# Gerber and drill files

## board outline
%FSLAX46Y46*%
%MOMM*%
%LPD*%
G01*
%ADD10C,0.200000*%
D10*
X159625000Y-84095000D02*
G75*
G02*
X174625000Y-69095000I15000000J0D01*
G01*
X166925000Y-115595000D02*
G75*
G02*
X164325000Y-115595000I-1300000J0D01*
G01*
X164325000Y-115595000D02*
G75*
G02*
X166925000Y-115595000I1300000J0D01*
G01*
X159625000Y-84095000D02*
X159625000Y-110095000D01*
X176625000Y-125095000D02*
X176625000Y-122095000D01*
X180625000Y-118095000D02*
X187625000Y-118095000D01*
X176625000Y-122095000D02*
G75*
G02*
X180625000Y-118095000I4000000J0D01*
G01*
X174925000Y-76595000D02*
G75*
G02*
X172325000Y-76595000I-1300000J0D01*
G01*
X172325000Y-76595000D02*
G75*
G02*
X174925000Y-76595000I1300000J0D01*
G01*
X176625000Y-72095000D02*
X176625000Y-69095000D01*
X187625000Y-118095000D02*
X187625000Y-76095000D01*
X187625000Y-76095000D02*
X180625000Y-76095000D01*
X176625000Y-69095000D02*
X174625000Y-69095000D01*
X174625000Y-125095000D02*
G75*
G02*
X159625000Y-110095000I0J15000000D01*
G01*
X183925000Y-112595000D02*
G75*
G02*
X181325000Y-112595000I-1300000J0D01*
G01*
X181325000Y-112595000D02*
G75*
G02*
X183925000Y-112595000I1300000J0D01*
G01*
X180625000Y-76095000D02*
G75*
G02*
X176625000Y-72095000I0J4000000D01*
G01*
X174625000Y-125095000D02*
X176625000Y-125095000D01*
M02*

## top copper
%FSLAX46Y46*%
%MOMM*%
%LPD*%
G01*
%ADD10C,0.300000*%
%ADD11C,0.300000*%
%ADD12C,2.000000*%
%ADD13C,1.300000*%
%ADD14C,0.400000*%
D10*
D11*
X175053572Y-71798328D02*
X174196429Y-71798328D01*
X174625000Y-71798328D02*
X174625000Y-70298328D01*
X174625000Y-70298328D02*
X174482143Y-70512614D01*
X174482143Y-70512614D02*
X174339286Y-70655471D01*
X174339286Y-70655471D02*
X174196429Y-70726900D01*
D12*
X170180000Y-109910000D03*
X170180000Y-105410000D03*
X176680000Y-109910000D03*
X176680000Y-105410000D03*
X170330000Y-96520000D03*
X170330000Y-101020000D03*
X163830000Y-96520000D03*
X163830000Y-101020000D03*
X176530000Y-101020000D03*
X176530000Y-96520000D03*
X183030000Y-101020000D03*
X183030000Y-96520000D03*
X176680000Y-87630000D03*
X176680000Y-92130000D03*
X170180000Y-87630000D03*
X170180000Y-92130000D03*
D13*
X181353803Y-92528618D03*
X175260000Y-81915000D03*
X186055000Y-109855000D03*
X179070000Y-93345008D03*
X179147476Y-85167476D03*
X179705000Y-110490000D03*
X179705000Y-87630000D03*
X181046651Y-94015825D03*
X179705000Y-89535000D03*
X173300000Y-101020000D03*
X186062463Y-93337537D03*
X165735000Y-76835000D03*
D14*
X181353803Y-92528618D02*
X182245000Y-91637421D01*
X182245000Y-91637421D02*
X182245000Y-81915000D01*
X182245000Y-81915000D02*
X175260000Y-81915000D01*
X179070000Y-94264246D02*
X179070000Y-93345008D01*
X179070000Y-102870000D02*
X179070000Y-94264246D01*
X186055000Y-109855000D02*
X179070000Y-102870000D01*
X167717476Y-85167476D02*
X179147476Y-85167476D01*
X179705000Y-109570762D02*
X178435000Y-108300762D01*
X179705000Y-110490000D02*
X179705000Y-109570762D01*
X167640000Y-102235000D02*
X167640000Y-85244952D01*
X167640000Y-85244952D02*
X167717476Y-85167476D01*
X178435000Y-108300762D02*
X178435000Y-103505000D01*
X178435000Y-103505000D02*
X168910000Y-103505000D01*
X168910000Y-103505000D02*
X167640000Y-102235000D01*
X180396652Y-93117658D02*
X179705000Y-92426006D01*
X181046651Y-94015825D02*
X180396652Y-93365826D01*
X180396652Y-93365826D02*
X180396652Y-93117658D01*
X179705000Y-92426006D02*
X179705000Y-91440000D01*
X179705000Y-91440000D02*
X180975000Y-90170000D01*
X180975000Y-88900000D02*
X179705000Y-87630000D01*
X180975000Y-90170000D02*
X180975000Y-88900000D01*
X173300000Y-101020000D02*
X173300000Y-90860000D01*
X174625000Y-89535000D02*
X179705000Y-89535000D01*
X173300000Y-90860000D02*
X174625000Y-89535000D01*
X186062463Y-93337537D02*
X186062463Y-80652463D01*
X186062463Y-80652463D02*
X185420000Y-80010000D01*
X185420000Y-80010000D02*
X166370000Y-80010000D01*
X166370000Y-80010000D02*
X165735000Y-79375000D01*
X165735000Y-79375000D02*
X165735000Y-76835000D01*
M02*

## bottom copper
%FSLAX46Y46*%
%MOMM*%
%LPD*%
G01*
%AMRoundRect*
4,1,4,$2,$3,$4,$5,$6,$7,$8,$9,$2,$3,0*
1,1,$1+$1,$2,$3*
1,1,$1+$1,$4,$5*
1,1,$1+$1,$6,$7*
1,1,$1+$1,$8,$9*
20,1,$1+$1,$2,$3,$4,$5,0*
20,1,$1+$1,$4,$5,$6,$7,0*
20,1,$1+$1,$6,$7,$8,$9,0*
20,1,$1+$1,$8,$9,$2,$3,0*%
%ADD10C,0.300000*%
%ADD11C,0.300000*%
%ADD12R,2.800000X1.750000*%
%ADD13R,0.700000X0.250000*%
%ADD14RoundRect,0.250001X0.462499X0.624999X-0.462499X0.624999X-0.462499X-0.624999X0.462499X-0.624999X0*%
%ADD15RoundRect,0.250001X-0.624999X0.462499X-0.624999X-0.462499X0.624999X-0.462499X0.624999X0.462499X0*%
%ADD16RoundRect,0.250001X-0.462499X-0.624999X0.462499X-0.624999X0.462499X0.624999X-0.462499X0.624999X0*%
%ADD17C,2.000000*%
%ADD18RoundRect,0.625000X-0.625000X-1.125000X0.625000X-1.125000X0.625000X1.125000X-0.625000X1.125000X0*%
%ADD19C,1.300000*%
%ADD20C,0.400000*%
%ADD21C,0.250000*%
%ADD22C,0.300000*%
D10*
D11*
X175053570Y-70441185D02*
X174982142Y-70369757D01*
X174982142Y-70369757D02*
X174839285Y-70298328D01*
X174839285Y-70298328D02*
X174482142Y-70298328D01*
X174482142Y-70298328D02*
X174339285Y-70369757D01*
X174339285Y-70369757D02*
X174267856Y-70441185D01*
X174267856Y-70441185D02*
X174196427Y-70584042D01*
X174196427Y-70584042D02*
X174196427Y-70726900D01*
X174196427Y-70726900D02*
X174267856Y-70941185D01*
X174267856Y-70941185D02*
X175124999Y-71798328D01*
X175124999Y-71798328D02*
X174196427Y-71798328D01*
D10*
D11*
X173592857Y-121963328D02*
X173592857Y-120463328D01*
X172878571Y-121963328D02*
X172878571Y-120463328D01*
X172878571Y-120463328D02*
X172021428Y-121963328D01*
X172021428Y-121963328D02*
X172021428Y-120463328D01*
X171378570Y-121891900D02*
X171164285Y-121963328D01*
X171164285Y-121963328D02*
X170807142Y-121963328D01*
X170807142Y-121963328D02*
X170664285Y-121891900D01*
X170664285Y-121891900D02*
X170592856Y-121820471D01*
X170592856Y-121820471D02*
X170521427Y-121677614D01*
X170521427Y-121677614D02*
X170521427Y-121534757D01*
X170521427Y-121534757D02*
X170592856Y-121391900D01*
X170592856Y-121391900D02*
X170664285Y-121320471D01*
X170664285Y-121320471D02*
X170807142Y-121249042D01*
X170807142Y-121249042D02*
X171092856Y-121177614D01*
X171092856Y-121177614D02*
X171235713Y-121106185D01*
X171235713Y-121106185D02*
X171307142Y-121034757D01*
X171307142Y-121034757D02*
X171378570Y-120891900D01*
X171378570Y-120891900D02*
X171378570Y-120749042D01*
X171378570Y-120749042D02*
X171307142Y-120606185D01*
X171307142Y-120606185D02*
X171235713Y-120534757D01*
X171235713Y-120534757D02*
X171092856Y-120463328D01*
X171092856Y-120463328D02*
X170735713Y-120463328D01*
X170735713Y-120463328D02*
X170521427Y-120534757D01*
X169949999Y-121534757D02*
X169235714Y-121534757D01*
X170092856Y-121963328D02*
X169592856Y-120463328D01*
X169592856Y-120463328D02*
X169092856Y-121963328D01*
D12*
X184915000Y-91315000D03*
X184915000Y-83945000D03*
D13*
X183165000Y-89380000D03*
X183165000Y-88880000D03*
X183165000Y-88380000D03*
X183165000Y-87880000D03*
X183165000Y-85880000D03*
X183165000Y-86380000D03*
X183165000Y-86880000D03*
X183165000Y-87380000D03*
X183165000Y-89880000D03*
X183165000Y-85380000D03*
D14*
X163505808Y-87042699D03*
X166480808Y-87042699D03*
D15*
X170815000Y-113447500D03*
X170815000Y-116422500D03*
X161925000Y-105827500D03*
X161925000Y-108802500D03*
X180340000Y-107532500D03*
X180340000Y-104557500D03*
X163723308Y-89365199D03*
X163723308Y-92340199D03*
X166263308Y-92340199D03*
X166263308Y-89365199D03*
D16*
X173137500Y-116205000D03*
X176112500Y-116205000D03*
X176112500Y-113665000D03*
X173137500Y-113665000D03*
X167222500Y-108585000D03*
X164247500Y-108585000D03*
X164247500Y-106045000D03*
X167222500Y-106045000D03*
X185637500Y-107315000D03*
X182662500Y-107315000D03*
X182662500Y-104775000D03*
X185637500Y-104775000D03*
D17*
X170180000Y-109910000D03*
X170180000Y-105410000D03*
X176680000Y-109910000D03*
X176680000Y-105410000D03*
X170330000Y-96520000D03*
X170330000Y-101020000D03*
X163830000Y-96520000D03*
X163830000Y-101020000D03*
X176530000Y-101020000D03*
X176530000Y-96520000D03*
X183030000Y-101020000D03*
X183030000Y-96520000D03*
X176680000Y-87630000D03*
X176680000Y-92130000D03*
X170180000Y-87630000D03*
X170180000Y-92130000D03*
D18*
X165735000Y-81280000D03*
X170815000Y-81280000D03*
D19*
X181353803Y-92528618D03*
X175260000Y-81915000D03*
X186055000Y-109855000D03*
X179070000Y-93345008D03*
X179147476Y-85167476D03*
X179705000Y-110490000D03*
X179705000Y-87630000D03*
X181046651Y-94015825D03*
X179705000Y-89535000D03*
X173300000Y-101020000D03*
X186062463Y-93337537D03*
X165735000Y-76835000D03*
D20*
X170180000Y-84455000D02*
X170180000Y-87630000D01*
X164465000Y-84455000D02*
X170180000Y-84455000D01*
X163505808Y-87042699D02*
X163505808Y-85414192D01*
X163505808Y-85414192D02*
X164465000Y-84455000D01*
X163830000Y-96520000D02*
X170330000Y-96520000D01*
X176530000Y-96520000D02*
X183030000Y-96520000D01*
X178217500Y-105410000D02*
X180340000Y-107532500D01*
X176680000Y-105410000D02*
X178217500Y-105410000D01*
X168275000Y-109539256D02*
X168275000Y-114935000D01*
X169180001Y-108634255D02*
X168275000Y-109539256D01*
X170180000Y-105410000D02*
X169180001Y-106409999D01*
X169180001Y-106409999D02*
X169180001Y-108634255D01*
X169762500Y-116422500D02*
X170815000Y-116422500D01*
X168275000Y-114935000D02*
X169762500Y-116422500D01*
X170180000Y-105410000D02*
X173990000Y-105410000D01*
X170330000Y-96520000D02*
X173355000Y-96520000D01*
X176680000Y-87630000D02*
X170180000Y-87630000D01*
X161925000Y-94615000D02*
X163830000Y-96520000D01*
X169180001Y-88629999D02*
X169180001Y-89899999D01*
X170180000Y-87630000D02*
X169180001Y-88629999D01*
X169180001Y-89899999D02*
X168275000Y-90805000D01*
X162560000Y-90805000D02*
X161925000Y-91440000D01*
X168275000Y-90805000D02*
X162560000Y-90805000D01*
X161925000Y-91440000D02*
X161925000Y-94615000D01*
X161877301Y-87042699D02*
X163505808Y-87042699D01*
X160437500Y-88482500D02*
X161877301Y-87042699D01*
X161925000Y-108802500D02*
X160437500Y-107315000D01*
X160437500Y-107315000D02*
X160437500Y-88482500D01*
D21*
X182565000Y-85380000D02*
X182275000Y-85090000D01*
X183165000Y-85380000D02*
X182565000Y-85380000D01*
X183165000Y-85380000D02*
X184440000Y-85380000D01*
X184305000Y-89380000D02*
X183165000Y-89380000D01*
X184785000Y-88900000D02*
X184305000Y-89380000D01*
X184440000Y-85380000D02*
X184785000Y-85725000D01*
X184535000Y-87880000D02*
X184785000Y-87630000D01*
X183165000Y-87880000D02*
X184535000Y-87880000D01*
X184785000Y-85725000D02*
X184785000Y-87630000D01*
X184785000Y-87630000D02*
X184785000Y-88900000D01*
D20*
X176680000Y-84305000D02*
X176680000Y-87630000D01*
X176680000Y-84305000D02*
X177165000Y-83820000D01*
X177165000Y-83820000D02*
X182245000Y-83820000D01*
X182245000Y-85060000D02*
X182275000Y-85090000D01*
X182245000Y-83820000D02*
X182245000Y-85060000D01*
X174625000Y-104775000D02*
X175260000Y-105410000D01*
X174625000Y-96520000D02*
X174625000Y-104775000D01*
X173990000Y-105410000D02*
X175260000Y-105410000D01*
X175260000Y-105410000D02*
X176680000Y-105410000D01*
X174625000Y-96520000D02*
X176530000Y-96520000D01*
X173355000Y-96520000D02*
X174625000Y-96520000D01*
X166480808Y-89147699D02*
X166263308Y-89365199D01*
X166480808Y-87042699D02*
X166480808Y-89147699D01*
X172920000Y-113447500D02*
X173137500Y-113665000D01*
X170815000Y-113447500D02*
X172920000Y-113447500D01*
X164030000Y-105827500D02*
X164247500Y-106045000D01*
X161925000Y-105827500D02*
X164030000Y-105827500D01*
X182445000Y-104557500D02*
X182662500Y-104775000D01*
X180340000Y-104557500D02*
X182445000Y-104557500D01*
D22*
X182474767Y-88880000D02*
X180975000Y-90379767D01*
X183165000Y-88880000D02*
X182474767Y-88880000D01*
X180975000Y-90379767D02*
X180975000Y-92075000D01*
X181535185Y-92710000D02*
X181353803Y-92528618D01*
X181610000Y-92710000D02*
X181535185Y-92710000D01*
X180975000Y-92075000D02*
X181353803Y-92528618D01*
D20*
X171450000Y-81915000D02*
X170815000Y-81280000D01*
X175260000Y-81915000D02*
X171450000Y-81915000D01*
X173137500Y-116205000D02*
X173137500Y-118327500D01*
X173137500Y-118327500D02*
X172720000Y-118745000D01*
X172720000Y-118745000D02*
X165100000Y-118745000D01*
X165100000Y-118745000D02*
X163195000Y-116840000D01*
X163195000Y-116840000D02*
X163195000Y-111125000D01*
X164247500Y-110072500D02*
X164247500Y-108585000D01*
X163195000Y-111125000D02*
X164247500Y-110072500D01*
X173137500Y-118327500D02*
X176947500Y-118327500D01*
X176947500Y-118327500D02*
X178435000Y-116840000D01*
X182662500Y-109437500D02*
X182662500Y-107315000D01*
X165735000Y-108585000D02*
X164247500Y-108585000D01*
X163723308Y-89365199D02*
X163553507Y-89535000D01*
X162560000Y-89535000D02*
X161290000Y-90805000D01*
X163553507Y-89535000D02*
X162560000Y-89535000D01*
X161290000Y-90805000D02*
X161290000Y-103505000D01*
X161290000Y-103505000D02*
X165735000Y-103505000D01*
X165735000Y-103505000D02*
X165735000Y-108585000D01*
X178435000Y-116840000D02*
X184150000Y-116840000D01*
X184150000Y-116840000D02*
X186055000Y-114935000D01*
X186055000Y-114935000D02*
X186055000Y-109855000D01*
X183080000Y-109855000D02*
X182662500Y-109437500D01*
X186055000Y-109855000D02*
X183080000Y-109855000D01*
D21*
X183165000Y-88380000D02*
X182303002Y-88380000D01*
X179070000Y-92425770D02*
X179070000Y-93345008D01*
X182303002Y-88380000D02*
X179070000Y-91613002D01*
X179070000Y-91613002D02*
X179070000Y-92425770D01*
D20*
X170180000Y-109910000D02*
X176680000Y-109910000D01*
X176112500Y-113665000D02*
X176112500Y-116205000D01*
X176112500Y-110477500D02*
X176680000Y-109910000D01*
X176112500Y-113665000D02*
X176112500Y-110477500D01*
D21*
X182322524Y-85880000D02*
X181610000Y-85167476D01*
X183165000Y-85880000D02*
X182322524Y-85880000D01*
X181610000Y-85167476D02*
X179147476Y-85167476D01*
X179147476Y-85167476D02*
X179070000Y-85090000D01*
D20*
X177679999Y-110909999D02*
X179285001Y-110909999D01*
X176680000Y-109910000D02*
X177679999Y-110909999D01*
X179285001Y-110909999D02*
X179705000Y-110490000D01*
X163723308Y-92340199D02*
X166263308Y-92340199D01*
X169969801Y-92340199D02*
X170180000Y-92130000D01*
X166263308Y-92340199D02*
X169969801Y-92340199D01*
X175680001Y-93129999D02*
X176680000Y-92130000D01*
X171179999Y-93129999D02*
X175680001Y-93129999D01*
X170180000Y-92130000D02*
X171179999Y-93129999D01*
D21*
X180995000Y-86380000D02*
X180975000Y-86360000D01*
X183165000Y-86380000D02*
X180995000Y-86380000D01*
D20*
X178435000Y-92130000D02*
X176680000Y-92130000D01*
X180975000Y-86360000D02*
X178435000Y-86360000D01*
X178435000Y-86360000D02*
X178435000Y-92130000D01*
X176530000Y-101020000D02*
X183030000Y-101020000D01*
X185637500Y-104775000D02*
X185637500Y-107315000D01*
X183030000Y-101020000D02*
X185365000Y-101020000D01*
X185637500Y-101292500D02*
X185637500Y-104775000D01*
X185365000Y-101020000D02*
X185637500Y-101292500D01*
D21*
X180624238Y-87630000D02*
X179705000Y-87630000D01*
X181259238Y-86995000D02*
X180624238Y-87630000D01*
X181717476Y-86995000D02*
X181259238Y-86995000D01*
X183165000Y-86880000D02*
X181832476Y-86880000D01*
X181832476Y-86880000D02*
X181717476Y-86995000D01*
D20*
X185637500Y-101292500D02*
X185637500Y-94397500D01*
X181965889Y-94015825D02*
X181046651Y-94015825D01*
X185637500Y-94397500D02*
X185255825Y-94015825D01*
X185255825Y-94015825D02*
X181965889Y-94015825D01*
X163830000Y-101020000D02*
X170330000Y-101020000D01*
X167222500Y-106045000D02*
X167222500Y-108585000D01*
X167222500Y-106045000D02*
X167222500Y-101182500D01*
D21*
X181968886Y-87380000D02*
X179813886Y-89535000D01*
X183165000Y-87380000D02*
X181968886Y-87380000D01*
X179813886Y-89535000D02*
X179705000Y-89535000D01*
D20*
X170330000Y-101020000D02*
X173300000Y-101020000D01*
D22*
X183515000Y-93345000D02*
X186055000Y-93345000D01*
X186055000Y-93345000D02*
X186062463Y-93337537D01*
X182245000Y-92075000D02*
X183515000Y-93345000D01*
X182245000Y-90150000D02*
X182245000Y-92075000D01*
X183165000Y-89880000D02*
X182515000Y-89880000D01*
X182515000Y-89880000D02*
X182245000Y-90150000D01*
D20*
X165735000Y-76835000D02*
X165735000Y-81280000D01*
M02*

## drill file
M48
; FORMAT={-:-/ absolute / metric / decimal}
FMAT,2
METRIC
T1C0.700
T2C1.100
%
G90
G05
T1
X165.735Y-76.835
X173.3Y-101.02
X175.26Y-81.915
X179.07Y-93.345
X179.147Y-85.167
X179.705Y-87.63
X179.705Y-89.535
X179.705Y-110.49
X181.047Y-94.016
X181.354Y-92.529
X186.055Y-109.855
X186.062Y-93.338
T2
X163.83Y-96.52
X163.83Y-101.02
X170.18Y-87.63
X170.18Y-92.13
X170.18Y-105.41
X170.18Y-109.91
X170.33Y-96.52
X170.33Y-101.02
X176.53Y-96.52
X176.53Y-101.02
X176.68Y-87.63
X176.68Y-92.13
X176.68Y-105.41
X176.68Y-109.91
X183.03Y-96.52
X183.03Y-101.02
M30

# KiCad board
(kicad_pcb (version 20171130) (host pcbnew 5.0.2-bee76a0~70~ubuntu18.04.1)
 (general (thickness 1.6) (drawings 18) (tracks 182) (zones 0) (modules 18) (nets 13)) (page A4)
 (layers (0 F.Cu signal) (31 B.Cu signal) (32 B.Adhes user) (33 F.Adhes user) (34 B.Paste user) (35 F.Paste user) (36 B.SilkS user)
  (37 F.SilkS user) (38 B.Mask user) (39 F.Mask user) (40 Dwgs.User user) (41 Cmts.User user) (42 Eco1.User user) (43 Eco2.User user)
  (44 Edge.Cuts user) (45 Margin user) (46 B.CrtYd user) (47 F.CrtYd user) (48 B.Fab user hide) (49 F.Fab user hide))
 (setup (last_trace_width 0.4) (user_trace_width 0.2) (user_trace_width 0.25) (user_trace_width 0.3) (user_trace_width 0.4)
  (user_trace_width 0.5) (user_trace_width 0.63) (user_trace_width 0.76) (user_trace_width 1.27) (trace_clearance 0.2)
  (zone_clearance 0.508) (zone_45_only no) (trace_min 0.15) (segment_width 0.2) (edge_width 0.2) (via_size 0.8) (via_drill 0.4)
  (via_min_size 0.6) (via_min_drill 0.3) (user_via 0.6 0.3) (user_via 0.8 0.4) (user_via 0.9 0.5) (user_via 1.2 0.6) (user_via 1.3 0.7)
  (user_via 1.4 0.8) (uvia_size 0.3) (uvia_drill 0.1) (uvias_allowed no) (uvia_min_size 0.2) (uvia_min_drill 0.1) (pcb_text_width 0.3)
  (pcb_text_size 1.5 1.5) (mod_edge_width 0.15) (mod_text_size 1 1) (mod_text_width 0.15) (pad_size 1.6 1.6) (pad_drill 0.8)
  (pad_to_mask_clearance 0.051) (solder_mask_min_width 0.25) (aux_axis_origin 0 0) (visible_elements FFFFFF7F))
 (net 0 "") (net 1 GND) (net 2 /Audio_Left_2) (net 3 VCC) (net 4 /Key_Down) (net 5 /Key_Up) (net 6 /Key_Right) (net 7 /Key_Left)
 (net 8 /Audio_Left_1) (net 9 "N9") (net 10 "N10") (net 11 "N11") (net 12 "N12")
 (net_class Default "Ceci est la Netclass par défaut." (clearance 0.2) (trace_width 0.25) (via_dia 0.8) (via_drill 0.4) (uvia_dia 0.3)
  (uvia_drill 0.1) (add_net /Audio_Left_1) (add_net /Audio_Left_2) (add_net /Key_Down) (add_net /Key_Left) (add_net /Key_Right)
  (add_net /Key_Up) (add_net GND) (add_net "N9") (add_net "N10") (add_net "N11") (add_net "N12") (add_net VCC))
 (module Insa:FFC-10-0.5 (layer B.Cu) (at 183.515 87.63 90)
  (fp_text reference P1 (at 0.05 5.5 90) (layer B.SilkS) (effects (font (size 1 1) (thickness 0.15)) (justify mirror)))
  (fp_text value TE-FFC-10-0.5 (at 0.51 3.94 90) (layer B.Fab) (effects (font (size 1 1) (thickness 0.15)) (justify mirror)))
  (pad A smd rect (at -3.685 1.4 90) (size 1.75 2.8) (layers B.Cu B.Paste B.Mask))
  (pad B smd rect (at 3.685 1.4 90) (size 1.75 2.8) (layers B.Cu B.Paste B.Mask))
  (pad 2 smd rect (at -1.75 -0.35 90) (size 0.25 0.7) (layers B.Cu B.Paste B.Mask) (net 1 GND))
  (pad 3 smd rect (at -1.25 -0.35 90) (size 0.25 0.7) (layers B.Cu B.Paste B.Mask) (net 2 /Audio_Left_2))
  (pad 4 smd rect (at -0.75 -0.35 90) (size 0.25 0.7) (layers B.Cu B.Paste B.Mask) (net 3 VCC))
  (pad 5 smd rect (at -0.25 -0.35 90) (size 0.25 0.7) (layers B.Cu B.Paste B.Mask) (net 1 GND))
  (pad 9 smd rect (at 1.75 -0.35 90) (size 0.25 0.7) (layers B.Cu B.Paste B.Mask) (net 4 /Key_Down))
  (pad 8 smd rect (at 1.25 -0.35 90) (size 0.25 0.7) (layers B.Cu B.Paste B.Mask) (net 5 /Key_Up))
  (pad 7 smd rect (at 0.75 -0.35 90) (size 0.25 0.7) (layers B.Cu B.Paste B.Mask) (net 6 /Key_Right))
  (pad 6 smd rect (at 0.25 -0.35 90) (size 0.25 0.7) (layers B.Cu B.Paste B.Mask) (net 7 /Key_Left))
  (pad 1 smd rect (at -2.25 -0.35 90) (size 0.25 0.7) (layers B.Cu B.Paste B.Mask) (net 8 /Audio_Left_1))
  (pad 10 smd rect (at 2.25 -0.35 90) (size 0.25 0.7) (layers B.Cu B.Paste B.Mask) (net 1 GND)))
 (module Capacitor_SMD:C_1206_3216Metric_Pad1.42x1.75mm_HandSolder (layer B.Cu) (at 164.993308 87.042699 180)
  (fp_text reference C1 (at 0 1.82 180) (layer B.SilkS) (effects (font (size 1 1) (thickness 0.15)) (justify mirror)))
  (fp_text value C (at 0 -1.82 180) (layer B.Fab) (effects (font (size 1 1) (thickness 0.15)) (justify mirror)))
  (pad 2 smd roundrect (at 1.4875 0 180) (size 1.425 1.75) (layers B.Cu B.Paste B.Mask) (roundrect_rratio 0.175439) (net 1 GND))
  (pad 1 smd roundrect (at -1.4875 0 180) (size 1.425 1.75) (layers B.Cu B.Paste B.Mask) (roundrect_rratio 0.175439) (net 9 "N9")))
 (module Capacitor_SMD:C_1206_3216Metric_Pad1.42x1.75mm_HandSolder (layer B.Cu) (at 170.815 114.935 270)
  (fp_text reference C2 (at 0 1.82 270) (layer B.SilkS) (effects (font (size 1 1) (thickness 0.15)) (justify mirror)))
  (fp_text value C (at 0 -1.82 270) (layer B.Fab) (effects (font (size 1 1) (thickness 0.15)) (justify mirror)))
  (pad 1 smd roundrect (at -1.4875 0 270) (size 1.425 1.75) (layers B.Cu B.Paste B.Mask) (roundrect_rratio 0.175439) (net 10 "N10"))
  (pad 2 smd roundrect (at 1.4875 0 270) (size 1.425 1.75) (layers B.Cu B.Paste B.Mask) (roundrect_rratio 0.175439) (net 1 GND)))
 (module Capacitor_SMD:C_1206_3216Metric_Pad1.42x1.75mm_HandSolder (layer B.Cu) (at 161.925 107.315 270)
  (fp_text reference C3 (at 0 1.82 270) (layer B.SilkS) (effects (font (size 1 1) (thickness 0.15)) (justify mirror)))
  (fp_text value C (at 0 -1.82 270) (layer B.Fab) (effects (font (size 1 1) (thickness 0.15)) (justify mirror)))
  (pad 1 smd roundrect (at -1.4875 0 270) (size 1.425 1.75) (layers B.Cu B.Paste B.Mask) (roundrect_rratio 0.175439) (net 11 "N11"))
  (pad 2 smd roundrect (at 1.4875 0 270) (size 1.425 1.75) (layers B.Cu B.Paste B.Mask) (roundrect_rratio 0.175439) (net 1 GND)))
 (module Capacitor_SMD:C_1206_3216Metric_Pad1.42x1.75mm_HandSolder (layer B.Cu) (at 180.34 106.045 270)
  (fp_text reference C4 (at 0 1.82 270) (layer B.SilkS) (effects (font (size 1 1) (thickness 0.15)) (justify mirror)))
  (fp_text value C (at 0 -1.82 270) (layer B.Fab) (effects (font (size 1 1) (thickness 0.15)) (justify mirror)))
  (pad 2 smd roundrect (at 1.4875 0 270) (size 1.425 1.75) (layers B.Cu B.Paste B.Mask) (roundrect_rratio 0.175439) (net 1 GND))
  (pad 1 smd roundrect (at -1.4875 0 270) (size 1.425 1.75) (layers B.Cu B.Paste B.Mask) (roundrect_rratio 0.175439) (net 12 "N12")))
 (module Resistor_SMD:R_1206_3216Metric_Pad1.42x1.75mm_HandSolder (layer B.Cu) (at 163.723308 90.852699 270)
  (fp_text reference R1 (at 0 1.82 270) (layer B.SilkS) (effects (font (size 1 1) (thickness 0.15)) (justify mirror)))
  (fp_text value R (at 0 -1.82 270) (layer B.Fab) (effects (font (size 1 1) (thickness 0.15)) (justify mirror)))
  (pad 1 smd roundrect (at -1.4875 0 270) (size 1.425 1.75) (layers B.Cu B.Paste B.Mask) (roundrect_rratio 0.175439) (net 3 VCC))
  (pad 2 smd roundrect (at 1.4875 0 270) (size 1.425 1.75) (layers B.Cu B.Paste B.Mask) (roundrect_rratio 0.175439) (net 5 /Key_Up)))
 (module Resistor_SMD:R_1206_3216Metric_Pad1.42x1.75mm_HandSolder (layer B.Cu) (at 166.263308 90.852699 270)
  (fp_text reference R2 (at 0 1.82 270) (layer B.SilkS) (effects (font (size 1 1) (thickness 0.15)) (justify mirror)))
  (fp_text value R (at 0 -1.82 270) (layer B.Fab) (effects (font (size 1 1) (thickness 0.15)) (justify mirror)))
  (pad 2 smd roundrect (at 1.4875 0 270) (size 1.425 1.75) (layers B.Cu B.Paste B.Mask) (roundrect_rratio 0.175439) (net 5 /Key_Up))
  (pad 1 smd roundrect (at -1.4875 0 270) (size 1.425 1.75) (layers B.Cu B.Paste B.Mask) (roundrect_rratio 0.175439) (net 9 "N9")))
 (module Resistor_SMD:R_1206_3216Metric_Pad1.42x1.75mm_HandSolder (layer B.Cu) (at 174.625 116.205)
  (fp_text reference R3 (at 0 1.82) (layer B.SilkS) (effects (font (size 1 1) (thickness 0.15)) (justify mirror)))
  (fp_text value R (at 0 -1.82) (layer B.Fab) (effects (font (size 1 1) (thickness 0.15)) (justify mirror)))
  (pad 1 smd roundrect (at -1.4875 0) (size 1.425 1.75) (layers B.Cu B.Paste B.Mask) (roundrect_rratio 0.175439) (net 3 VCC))
  (pad 2 smd roundrect (at 1.4875 0) (size 1.425 1.75) (layers B.Cu B.Paste B.Mask) (roundrect_rratio 0.175439) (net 4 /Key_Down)))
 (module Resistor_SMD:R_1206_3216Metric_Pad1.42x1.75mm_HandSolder (layer B.Cu) (at 174.625 113.665)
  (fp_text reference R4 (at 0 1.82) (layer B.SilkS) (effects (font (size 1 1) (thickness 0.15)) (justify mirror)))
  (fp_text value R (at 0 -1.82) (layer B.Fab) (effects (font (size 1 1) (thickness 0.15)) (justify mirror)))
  (pad 2 smd roundrect (at 1.4875 0) (size 1.425 1.75) (layers B.Cu B.Paste B.Mask) (roundrect_rratio 0.175439) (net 4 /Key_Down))
  (pad 1 smd roundrect (at -1.4875 0) (size 1.425 1.75) (layers B.Cu B.Paste B.Mask) (roundrect_rratio 0.175439) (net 10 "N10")))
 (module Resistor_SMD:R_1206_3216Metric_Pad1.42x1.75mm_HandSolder (layer B.Cu) (at 165.735 108.585)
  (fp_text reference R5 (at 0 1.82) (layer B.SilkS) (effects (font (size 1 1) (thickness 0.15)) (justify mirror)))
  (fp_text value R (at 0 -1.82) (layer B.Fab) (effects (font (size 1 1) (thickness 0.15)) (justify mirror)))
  (pad 2 smd roundrect (at 1.4875 0) (size 1.425 1.75) (layers B.Cu B.Paste B.Mask) (roundrect_rratio 0.175439) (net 7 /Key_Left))
  (pad 1 smd roundrect (at -1.4875 0) (size 1.425 1.75) (layers B.Cu B.Paste B.Mask) (roundrect_rratio 0.175439) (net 3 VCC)))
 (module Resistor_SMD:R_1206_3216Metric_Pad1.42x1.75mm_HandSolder (layer B.Cu) (at 165.735 106.045)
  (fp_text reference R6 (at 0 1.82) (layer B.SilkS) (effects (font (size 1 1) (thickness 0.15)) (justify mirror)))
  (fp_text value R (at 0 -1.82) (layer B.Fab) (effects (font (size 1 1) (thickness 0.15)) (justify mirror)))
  (pad 1 smd roundrect (at -1.4875 0) (size 1.425 1.75) (layers B.Cu B.Paste B.Mask) (roundrect_rratio 0.175439) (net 11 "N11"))
  (pad 2 smd roundrect (at 1.4875 0) (size 1.425 1.75) (layers B.Cu B.Paste B.Mask) (roundrect_rratio 0.175439) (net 7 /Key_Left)))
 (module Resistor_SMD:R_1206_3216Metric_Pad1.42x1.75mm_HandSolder (layer B.Cu) (at 184.15 107.315)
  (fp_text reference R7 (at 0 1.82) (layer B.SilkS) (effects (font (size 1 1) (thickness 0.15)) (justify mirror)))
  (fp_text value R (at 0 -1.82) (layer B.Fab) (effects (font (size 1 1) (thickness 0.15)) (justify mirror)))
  (pad 2 smd roundrect (at 1.4875 0) (size 1.425 1.75) (layers B.Cu B.Paste B.Mask) (roundrect_rratio 0.175439) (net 6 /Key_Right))
  (pad 1 smd roundrect (at -1.4875 0) (size 1.425 1.75) (layers B.Cu B.Paste B.Mask) (roundrect_rratio 0.175439) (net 3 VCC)))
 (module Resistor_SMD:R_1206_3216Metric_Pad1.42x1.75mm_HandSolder (layer B.Cu) (at 184.15 104.775)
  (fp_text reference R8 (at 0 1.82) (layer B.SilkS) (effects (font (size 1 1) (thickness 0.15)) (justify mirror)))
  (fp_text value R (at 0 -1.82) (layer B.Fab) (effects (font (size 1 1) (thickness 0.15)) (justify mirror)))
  (pad 1 smd roundrect (at -1.4875 0) (size 1.425 1.75) (layers B.Cu B.Paste B.Mask) (roundrect_rratio 0.175439) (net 12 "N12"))
  (pad 2 smd roundrect (at 1.4875 0) (size 1.425 1.75) (layers B.Cu B.Paste B.Mask) (roundrect_rratio 0.175439) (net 6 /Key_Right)))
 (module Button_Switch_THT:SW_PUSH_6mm (layer F.Cu) (at 170.18 105.41)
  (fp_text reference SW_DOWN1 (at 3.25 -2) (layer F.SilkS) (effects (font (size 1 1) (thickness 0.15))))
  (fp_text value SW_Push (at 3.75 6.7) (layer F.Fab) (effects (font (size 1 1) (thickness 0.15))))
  (pad 2 thru_hole circle (at 0 4.5 90) (size 2 2) (drill 1.1) (layers *.Cu *.Mask) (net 4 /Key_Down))
  (pad 1 thru_hole circle (at 0 0 90) (size 2 2) (drill 1.1) (layers *.Cu *.Mask) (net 1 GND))
  (pad 2 thru_hole circle (at 6.5 4.5 90) (size 2 2) (drill 1.1) (layers *.Cu *.Mask) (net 4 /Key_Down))
  (pad 1 thru_hole circle (at 6.5 0 90) (size 2 2) (drill 1.1) (layers *.Cu *.Mask) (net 1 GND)))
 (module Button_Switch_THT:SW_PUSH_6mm (layer F.Cu) (at 163.83 96.52)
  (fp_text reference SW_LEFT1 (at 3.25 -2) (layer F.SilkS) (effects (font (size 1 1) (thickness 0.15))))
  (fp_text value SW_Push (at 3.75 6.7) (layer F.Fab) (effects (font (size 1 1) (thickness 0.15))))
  (pad 1 thru_hole circle (at 6.5 0 90) (size 2 2) (drill 1.1) (layers *.Cu *.Mask) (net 1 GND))
  (pad 2 thru_hole circle (at 6.5 4.5 90) (size 2 2) (drill 1.1) (layers *.Cu *.Mask) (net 7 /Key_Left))
  (pad 1 thru_hole circle (at 0 0 90) (size 2 2) (drill 1.1) (layers *.Cu *.Mask) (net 1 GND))
  (pad 2 thru_hole circle (at 0 4.5 90) (size 2 2) (drill 1.1) (layers *.Cu *.Mask) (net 7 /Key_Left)))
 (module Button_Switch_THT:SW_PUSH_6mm (layer F.Cu) (at 176.53 96.52)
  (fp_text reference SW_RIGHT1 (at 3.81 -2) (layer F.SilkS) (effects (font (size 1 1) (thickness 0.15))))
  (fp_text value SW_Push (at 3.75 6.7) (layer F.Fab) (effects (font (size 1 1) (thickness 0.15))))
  (pad 2 thru_hole circle (at 0 4.5 90) (size 2 2) (drill 1.1) (layers *.Cu *.Mask) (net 6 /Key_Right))
  (pad 1 thru_hole circle (at 0 0 90) (size 2 2) (drill 1.1) (layers *.Cu *.Mask) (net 1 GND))
  (pad 2 thru_hole circle (at 6.5 4.5 90) (size 2 2) (drill 1.1) (layers *.Cu *.Mask) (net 6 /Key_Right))
  (pad 1 thru_hole circle (at 6.5 0 90) (size 2 2) (drill 1.1) (layers *.Cu *.Mask) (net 1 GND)))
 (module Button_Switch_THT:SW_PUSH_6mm (layer F.Cu) (at 170.18 87.63)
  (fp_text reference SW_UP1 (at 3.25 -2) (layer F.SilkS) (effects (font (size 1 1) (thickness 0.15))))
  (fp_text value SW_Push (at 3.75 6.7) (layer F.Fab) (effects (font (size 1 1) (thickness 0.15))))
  (pad 1 thru_hole circle (at 6.5 0 90) (size 2 2) (drill 1.1) (layers *.Cu *.Mask) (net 1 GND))
  (pad 2 thru_hole circle (at 6.5 4.5 90) (size 2 2) (drill 1.1) (layers *.Cu *.Mask) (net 5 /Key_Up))
  (pad 1 thru_hole circle (at 0 0 90) (size 2 2) (drill 1.1) (layers *.Cu *.Mask) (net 1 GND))
  (pad 2 thru_hole circle (at 0 4.5 90) (size 2 2) (drill 1.1) (layers *.Cu *.Mask) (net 5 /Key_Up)))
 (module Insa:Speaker (layer B.Cu) (at 168.275 81.28)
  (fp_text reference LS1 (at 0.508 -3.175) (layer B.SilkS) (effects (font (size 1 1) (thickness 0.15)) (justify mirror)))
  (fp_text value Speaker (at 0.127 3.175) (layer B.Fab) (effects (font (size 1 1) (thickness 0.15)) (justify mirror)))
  (pad 1 smd roundrect (at -2.54 0) (size 2.5 3.5) (layers B.Cu B.Paste B.Mask) (roundrect_rratio 0.25) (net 8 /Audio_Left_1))
  (pad 2 smd roundrect (at 2.54 0) (size 2.5 3.5) (layers B.Cu B.Paste B.Mask) (roundrect_rratio 0.25) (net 2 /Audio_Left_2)))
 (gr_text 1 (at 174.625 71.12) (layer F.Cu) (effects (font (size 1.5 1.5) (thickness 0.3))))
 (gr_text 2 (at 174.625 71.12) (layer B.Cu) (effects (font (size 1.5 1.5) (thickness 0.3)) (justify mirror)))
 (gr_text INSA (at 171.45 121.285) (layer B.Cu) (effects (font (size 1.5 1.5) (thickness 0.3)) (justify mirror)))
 (gr_arc (start 174.625 84.095) (end 174.625 69.095) (angle -90) (layer Edge.Cuts) (width 0.2))
 (gr_circle (center 165.625 115.595) (end 166.925 115.595) (layer Edge.Cuts) (width 0.2))
 (gr_line (start 159.625 84.095) (end 159.625 110.095) (layer Edge.Cuts) (width 0.2))
 (gr_line (start 176.625 125.095) (end 176.625 122.095) (layer Edge.Cuts) (width 0.2))
 (gr_line (start 180.625 118.095) (end 187.625 118.095) (layer Edge.Cuts) (width 0.2))
 (gr_arc (start 180.625 122.095) (end 180.625 118.095) (angle -90) (layer Edge.Cuts) (width 0.2))
 (gr_circle (center 173.625 76.595) (end 174.925 76.595) (layer Edge.Cuts) (width 0.2))
 (gr_line (start 176.625 72.095) (end 176.625 69.095) (layer Edge.Cuts) (width 0.2))
 (gr_line (start 187.625 118.095) (end 187.625 76.095) (layer Edge.Cuts) (width 0.2))
 (gr_line (start 187.625 76.095) (end 180.625 76.095) (layer Edge.Cuts) (width 0.2))
 (gr_line (start 176.625 69.095) (end 174.625 69.095) (layer Edge.Cuts) (width 0.2))
 (gr_arc (start 174.625 110.095) (end 159.625 110.095) (angle -90) (layer Edge.Cuts) (width 0.2))
 (gr_circle (center 182.625 112.595) (end 183.925 112.595) (layer Edge.Cuts) (width 0.2))
 (gr_arc (start 180.625 72.095) (end 176.625 72.095) (angle -90) (layer Edge.Cuts) (width 0.2))
 (gr_line (start 174.625 125.095) (end 176.625 125.095) (layer Edge.Cuts) (width 0.2))
 (segment (start 170.18 84.455) (end 170.18 87.63) (width 0.4) (layer B.Cu) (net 1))
 (segment (start 164.465 84.455) (end 170.18 84.455) (width 0.4) (layer B.Cu) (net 1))
 (segment (start 163.505808 87.042699) (end 163.505808 85.414192) (width 0.4) (layer B.Cu) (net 1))
 (segment (start 163.505808 85.414192) (end 164.465 84.455) (width 0.4) (layer B.Cu) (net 1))
 (segment (start 163.83 96.52) (end 170.33 96.52) (width 0.4) (layer B.Cu) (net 1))
 (segment (start 176.53 96.52) (end 183.03 96.52) (width 0.4) (layer B.Cu) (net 1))
 (segment (start 178.2175 105.41) (end 180.34 107.5325) (width 0.4) (layer B.Cu) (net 1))
 (segment (start 176.68 105.41) (end 178.2175 105.41) (width 0.4) (layer B.Cu) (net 1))
 (segment (start 168.275 109.539256) (end 168.275 114.935) (width 0.4) (layer B.Cu) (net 1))
 (segment (start 169.180001 108.634255) (end 168.275 109.539256) (width 0.4) (layer B.Cu) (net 1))
 (segment (start 170.18 105.41) (end 169.180001 106.409999) (width 0.4) (layer B.Cu) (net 1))
 (segment (start 169.180001 106.409999) (end 169.180001 108.634255) (width 0.4) (layer B.Cu) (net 1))
 (segment (start 169.7625 116.4225) (end 170.815 116.4225) (width 0.4) (layer B.Cu) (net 1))
 (segment (start 168.275 114.935) (end 169.7625 116.4225) (width 0.4) (layer B.Cu) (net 1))
 (segment (start 170.18 105.41) (end 173.99 105.41) (width 0.4) (layer B.Cu) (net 1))
 (segment (start 170.33 96.52) (end 173.355 96.52) (width 0.4) (layer B.Cu) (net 1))
 (segment (start 176.68 87.63) (end 170.18 87.63) (width 0.4) (layer B.Cu) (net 1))
 (segment (start 161.925 94.615) (end 163.83 96.52) (width 0.4) (layer B.Cu) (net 1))
 (segment (start 169.180001 88.629999) (end 169.180001 89.899999) (width 0.4) (layer B.Cu) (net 1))
 (segment (start 170.18 87.63) (end 169.180001 88.629999) (width 0.4) (layer B.Cu) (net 1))
 (segment (start 169.180001 89.899999) (end 168.275 90.805) (width 0.4) (layer B.Cu) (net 1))
 (segment (start 162.56 90.805) (end 161.925 91.44) (width 0.4) (layer B.Cu) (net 1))
 (segment (start 168.275 90.805) (end 162.56 90.805) (width 0.4) (layer B.Cu) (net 1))
 (segment (start 161.925 91.44) (end 161.925 94.615) (width 0.4) (layer B.Cu) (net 1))
 (segment (start 161.877301 87.042699) (end 163.505808 87.042699) (width 0.4) (layer B.Cu) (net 1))
 (segment (start 160.4375 88.4825) (end 161.877301 87.042699) (width 0.4) (layer B.Cu) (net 1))
 (segment (start 161.925 108.8025) (end 160.4375 107.315) (width 0.4) (layer B.Cu) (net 1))
 (segment (start 160.4375 107.315) (end 160.4375 88.4825) (width 0.4) (layer B.Cu) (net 1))
 (segment (start 182.565 85.38) (end 182.275 85.09) (width 0.25) (layer B.Cu) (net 1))
 (segment (start 183.165 85.38) (end 182.565 85.38) (width 0.25) (layer B.Cu) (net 1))
 (segment (start 183.165 85.38) (end 184.44 85.38) (width 0.25) (layer B.Cu) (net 1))
 (segment (start 184.305 89.38) (end 183.165 89.38) (width 0.25) (layer B.Cu) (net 1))
 (segment (start 184.785 88.9) (end 184.305 89.38) (width 0.25) (layer B.Cu) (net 1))
 (segment (start 184.44 85.38) (end 184.785 85.725) (width 0.25) (layer B.Cu) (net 1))
 (segment (start 184.535 87.88) (end 184.785 87.63) (width 0.25) (layer B.Cu) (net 1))
 (segment (start 183.165 87.88) (end 184.535 87.88) (width 0.25) (layer B.Cu) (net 1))
 (segment (start 184.785 85.725) (end 184.785 87.63) (width 0.25) (layer B.Cu) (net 1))
 (segment (start 184.785 87.63) (end 184.785 88.9) (width 0.25) (layer B.Cu) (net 1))
 (segment (start 176.68 84.305) (end 176.68 87.63) (width 0.4) (layer B.Cu) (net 1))
 (segment (start 176.68 84.305) (end 177.165 83.82) (width 0.4) (layer B.Cu) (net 1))
 (segment (start 177.165 83.82) (end 182.245 83.82) (width 0.4) (layer B.Cu) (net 1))
 (segment (start 182.245 85.06) (end 182.275 85.09) (width 0.4) (layer B.Cu) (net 1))
 (segment (start 182.245 83.82) (end 182.245 85.06) (width 0.4) (layer B.Cu) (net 1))
 (segment (start 174.625 104.775) (end 175.26 105.41) (width 0.4) (layer B.Cu) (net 1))
 (segment (start 174.625 96.52) (end 174.625 104.775) (width 0.4) (layer B.Cu) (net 1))
 (segment (start 173.99 105.41) (end 175.26 105.41) (width 0.4) (layer B.Cu) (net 1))
 (segment (start 175.26 105.41) (end 176.68 105.41) (width 0.4) (layer B.Cu) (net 1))
 (segment (start 174.625 96.52) (end 176.53 96.52) (width 0.4) (layer B.Cu) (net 1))
 (segment (start 173.355 96.52) (end 174.625 96.52) (width 0.4) (layer B.Cu) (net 1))
 (segment (start 166.480808 89.147699) (end 166.263308 89.365199) (width 0.4) (layer B.Cu) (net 9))
 (segment (start 166.480808 87.042699) (end 166.480808 89.147699) (width 0.4) (layer B.Cu) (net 9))
 (segment (start 172.92 113.4475) (end 173.1375 113.665) (width 0.4) (layer B.Cu) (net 10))
 (segment (start 170.815 113.4475) (end 172.92 113.4475) (width 0.4) (layer B.Cu) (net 10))
 (segment (start 164.03 105.8275) (end 164.2475 106.045) (width 0.4) (layer B.Cu) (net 11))
 (segment (start 161.925 105.8275) (end 164.03 105.8275) (width 0.4) (layer B.Cu) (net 11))
 (segment (start 182.445 104.5575) (end 182.6625 104.775) (width 0.4) (layer B.Cu) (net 12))
 (segment (start 180.34 104.5575) (end 182.445 104.5575) (width 0.4) (layer B.Cu) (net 12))
 (segment (start 182.474767 88.88) (end 180.975 90.379767) (width 0.3) (layer B.Cu) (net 2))
 (segment (start 183.165 88.88) (end 182.474767 88.88) (width 0.3) (layer B.Cu) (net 2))
 (segment (start 180.975 90.379767) (end 180.975 92.075) (width 0.3) (layer B.Cu) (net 2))
 (via (at 181.353803 92.528618) (size 1.3) (drill 0.7) (layers F.Cu B.Cu) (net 2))
 (segment (start 181.535185 92.71) (end 181.353803 92.528618) (width 0.3) (layer B.Cu) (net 2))
 (segment (start 181.61 92.71) (end 181.535185 92.71) (width 0.3) (layer B.Cu) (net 2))
 (segment (start 180.975 92.075) (end 181.353803 92.528618) (width 0.3) (layer B.Cu) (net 2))
 (segment (start 181.353803 92.528618) (end 182.245 91.637421) (width 0.4) (layer F.Cu) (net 2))
 (segment (start 182.245 91.637421) (end 182.245 81.915) (width 0.4) (layer F.Cu) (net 2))
 (segment (start 182.245 81.915) (end 175.26 81.915) (width 0.4) (layer F.Cu) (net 2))
 (via (at 175.26 81.915) (size 1.3) (drill 0.7) (layers F.Cu B.Cu) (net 2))
 (segment (start 171.45 81.915) (end 170.815 81.28) (width 0.4) (layer B.Cu) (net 2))
 (segment (start 175.26 81.915) (end 171.45 81.915) (width 0.4) (layer B.Cu) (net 2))
 (segment (start 173.1375 116.205) (end 173.1375 118.3275) (width 0.4) (layer B.Cu) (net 3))
 (segment (start 173.1375 118.3275) (end 172.72 118.745) (width 0.4) (layer B.Cu) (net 3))
 (segment (start 172.72 118.745) (end 165.1 118.745) (width 0.4) (layer B.Cu) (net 3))
 (segment (start 165.1 118.745) (end 163.195 116.84) (width 0.4) (layer B.Cu) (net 3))
 (segment (start 163.195 116.84) (end 163.195 111.125) (width 0.4) (layer B.Cu) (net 3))
 (segment (start 164.2475 110.0725) (end 164.2475 108.585) (width 0.4) (layer B.Cu) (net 3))
 (segment (start 163.195 111.125) (end 164.2475 110.0725) (width 0.4) (layer B.Cu) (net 3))
 (segment (start 173.1375 118.3275) (end 176.9475 118.3275) (width 0.4) (layer B.Cu) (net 3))
 (segment (start 176.9475 118.3275) (end 178.435 116.84) (width 0.4) (layer B.Cu) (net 3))
 (segment (start 182.6625 109.4375) (end 182.6625 107.315) (width 0.4) (layer B.Cu) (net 3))
 (segment (start 165.735 108.585) (end 164.2475 108.585) (width 0.4) (layer B.Cu) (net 3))
 (segment (start 163.723308 89.365199) (end 163.553507 89.535) (width 0.4) (layer B.Cu) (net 3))
 (segment (start 162.56 89.535) (end 161.29 90.805) (width 0.4) (layer B.Cu) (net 3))
 (segment (start 163.553507 89.535) (end 162.56 89.535) (width 0.4) (layer B.Cu) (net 3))
 (segment (start 161.29 90.805) (end 161.29 103.505) (width 0.4) (layer B.Cu) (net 3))
 (segment (start 161.29 103.505) (end 165.735 103.505) (width 0.4) (layer B.Cu) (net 3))
 (segment (start 165.735 103.505) (end 165.735 108.585) (width 0.4) (layer B.Cu) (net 3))
 (segment (start 178.435 116.84) (end 184.15 116.84) (width 0.4) (layer B.Cu) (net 3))
 (segment (start 184.15 116.84) (end 186.055 114.935) (width 0.4) (layer B.Cu) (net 3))
 (segment (start 186.055 114.935) (end 186.055 109.855) (width 0.4) (layer B.Cu) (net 3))
 (segment (start 183.08 109.855) (end 182.6625 109.4375) (width 0.4) (layer B.Cu) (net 3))
 (segment (start 186.055 109.855) (end 183.08 109.855) (width 0.4) (layer B.Cu) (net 3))
 (via (at 186.055 109.855) (size 1.3) (drill 0.7) (layers F.Cu B.Cu) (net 3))
 (via (at 179.07 93.345008) (size 1.3) (drill 0.7) (layers F.Cu B.Cu) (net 3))
 (segment (start 183.165 88.38) (end 182.303002 88.38) (width 0.25) (layer B.Cu) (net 3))
 (segment (start 179.07 92.42577) (end 179.07 93.345008) (width 0.25) (layer B.Cu) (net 3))
 (segment (start 182.303002 88.38) (end 179.07 91.613002) (width 0.25) (layer B.Cu) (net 3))
 (segment (start 179.07 94.264246) (end 179.07 93.345008) (width 0.4) (layer F.Cu) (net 3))
 (segment (start 179.07 102.87) (end 179.07 94.264246) (width 0.4) (layer F.Cu) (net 3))
 (segment (start 186.055 109.855) (end 179.07 102.87) (width 0.4) (layer F.Cu) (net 3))
 (segment (start 179.07 91.613002) (end 179.07 92.42577) (width 0.25) (layer B.Cu) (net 3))
 (segment (start 170.18 109.91) (end 176.68 109.91) (width 0.4) (layer B.Cu) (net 4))
 (segment (start 176.1125 113.665) (end 176.1125 116.205) (width 0.4) (layer B.Cu) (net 4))
 (segment (start 176.1125 110.4775) (end 176.68 109.91) (width 0.4) (layer B.Cu) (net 4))
 (segment (start 176.1125 113.665) (end 176.1125 110.4775) (width 0.4) (layer B.Cu) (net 4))
 (segment (start 182.322524 85.88) (end 181.61 85.167476) (width 0.25) (layer B.Cu) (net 4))
 (segment (start 183.165 85.88) (end 182.322524 85.88) (width 0.25) (layer B.Cu) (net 4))
 (segment (start 181.61 85.167476) (end 179.147476 85.167476) (width 0.25) (layer B.Cu) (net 4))
 (segment (start 179.147476 85.167476) (end 179.07 85.09) (width 0.25) (layer B.Cu) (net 4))
 (via (at 179.147476 85.167476) (size 1.3) (drill 0.7) (layers F.Cu B.Cu) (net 4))
 (segment (start 177.679999 110.909999) (end 179.285001 110.909999) (width 0.4) (layer B.Cu) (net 4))
 (segment (start 176.68 109.91) (end 177.679999 110.909999) (width 0.4) (layer B.Cu) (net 4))
 (via (at 179.705 110.49) (size 1.3) (drill 0.7) (layers F.Cu B.Cu) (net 4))
 (segment (start 179.285001 110.909999) (end 179.705 110.49) (width 0.4) (layer B.Cu) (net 4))
 (segment (start 167.717476 85.167476) (end 179.147476 85.167476) (width 0.4) (layer F.Cu) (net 4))
 (segment (start 179.705 109.570762) (end 178.435 108.300762) (width 0.4) (layer F.Cu) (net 4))
 (segment (start 179.705 110.49) (end 179.705 109.570762) (width 0.4) (layer F.Cu) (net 4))
 (segment (start 167.64 102.235) (end 167.64 85.244952) (width 0.4) (layer F.Cu) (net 4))
 (segment (start 167.64 85.244952) (end 167.717476 85.167476) (width 0.4) (layer F.Cu) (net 4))
 (segment (start 178.435 108.300762) (end 178.435 103.505) (width 0.4) (layer F.Cu) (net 4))
 (segment (start 178.435 103.505) (end 168.91 103.505) (width 0.4) (layer F.Cu) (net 4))
 (segment (start 168.91 103.505) (end 167.64 102.235) (width 0.4) (layer F.Cu) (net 4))
 (segment (start 163.723308 92.340199) (end 166.263308 92.340199) (width 0.4) (layer B.Cu) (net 5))
 (segment (start 169.969801 92.340199) (end 170.18 92.13) (width 0.4) (layer B.Cu) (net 5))
 (segment (start 166.263308 92.340199) (end 169.969801 92.340199) (width 0.4) (layer B.Cu) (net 5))
 (segment (start 175.680001 93.129999) (end 176.68 92.13) (width 0.4) (layer B.Cu) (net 5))
 (segment (start 171.179999 93.129999) (end 175.680001 93.129999) (width 0.4) (layer B.Cu) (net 5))
 (segment (start 170.18 92.13) (end 171.179999 93.129999) (width 0.4) (layer B.Cu) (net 5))
 (segment (start 180.995 86.38) (end 180.975 86.36) (width 0.25) (layer B.Cu) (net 5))
 (segment (start 183.165 86.38) (end 180.995 86.38) (width 0.25) (layer B.Cu) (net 5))
 (segment (start 178.435 92.13) (end 176.68 92.13) (width 0.4) (layer B.Cu) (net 5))
 (segment (start 180.975 86.36) (end 178.435 86.36) (width 0.4) (layer B.Cu) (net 5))
 (segment (start 178.435 86.36) (end 178.435 92.13) (width 0.4) (layer B.Cu) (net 5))
 (segment (start 176.53 101.02) (end 183.03 101.02) (width 0.4) (layer B.Cu) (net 6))
 (segment (start 185.6375 104.775) (end 185.6375 107.315) (width 0.4) (layer B.Cu) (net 6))
 (segment (start 183.03 101.02) (end 185.365 101.02) (width 0.4) (layer B.Cu) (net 6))
 (segment (start 185.6375 101.2925) (end 185.6375 104.775) (width 0.4) (layer B.Cu) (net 6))
 (segment (start 185.365 101.02) (end 185.6375 101.2925) (width 0.4) (layer B.Cu) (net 6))
 (via (at 179.705 87.63) (size 1.3) (drill 0.7) (layers F.Cu B.Cu) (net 6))
 (segment (start 180.624238 87.63) (end 179.705 87.63) (width 0.25) (layer B.Cu) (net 6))
 (segment (start 181.259238 86.995) (end 180.624238 87.63) (width 0.25) (layer B.Cu) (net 6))
 (segment (start 181.717476 86.995) (end 181.259238 86.995) (width 0.25) (layer B.Cu) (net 6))
 (segment (start 183.165 86.88) (end 181.832476 86.88) (width 0.25) (layer B.Cu) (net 6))
 (segment (start 181.832476 86.88) (end 181.717476 86.995) (width 0.25) (layer B.Cu) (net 6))
 (segment (start 185.6375 101.2925) (end 185.6375 94.3975) (width 0.4) (layer B.Cu) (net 6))
 (segment (start 181.965889 94.015825) (end 181.046651 94.015825) (width 0.4) (layer B.Cu) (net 6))
 (segment (start 185.6375 94.3975) (end 185.255825 94.015825) (width 0.4) (layer B.Cu) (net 6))
 (segment (start 185.255825 94.015825) (end 181.965889 94.015825) (width 0.4) (layer B.Cu) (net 6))
 (via (at 181.046651 94.015825) (size 1.3) (drill 0.7) (layers F.Cu B.Cu) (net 6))
 (segment (start 180.396652 93.117658) (end 179.705 92.426006) (width 0.4) (layer F.Cu) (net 6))
 (segment (start 181.046651 94.015825) (end 180.396652 93.365826) (width 0.4) (layer F.Cu) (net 6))
 (segment (start 180.396652 93.365826) (end 180.396652 93.117658) (width 0.4) (layer F.Cu) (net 6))
 (segment (start 179.705 92.426006) (end 179.705 91.44) (width 0.4) (layer F.Cu) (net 6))
 (segment (start 179.705 91.44) (end 180.975 90.17) (width 0.4) (layer F.Cu) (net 6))
 (segment (start 180.975 88.9) (end 179.705 87.63) (width 0.4) (layer F.Cu) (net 6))
 (segment (start 180.975 90.17) (end 180.975 88.9) (width 0.4) (layer F.Cu) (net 6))
 (segment (start 163.83 101.02) (end 170.33 101.02) (width 0.4) (layer B.Cu) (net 7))
 (segment (start 167.2225 106.045) (end 167.2225 108.585) (width 0.4) (layer B.Cu) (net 7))
 (segment (start 167.2225 106.045) (end 167.2225 101.1825) (width 0.4) (layer B.Cu) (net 7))
 (segment (start 181.968886 87.38) (end 179.813886 89.535) (width 0.25) (layer B.Cu) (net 7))
 (segment (start 183.165 87.38) (end 181.968886 87.38) (width 0.25) (layer B.Cu) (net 7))
 (segment (start 179.813886 89.535) (end 179.705 89.535) (width 0.25) (layer B.Cu) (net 7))
 (via (at 179.705 89.535) (size 1.3) (drill 0.7) (layers F.Cu B.Cu) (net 7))
 (segment (start 170.33 101.02) (end 173.3 101.02) (width 0.4) (layer B.Cu) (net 7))
 (via (at 173.3 101.02) (size 1.3) (drill 0.7) (layers F.Cu B.Cu) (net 7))
 (segment (start 173.3 101.02) (end 173.3 90.86) (width 0.4) (layer F.Cu) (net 7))
 (segment (start 174.625 89.535) (end 179.705 89.535) (width 0.4) (layer F.Cu) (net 7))
 (segment (start 173.3 90.86) (end 174.625 89.535) (width 0.4) (layer F.Cu) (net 7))
 (via (at 186.062463 93.337537) (size 1.3) (drill 0.7) (layers F.Cu B.Cu) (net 8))
 (segment (start 183.515 93.345) (end 186.055 93.345) (width 0.3) (layer B.Cu) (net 8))
 (segment (start 186.055 93.345) (end 186.062463 93.337537) (width 0.3) (layer B.Cu) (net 8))
 (segment (start 182.245 92.075) (end 183.515 93.345) (width 0.3) (layer B.Cu) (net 8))
 (segment (start 182.245 90.15) (end 182.245 92.075) (width 0.3) (layer B.Cu) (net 8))
 (segment (start 183.165 89.88) (end 182.515 89.88) (width 0.3) (layer B.Cu) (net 8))
 (segment (start 182.515 89.88) (end 182.245 90.15) (width 0.3) (layer B.Cu) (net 8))
 (segment (start 186.062463 93.337537) (end 186.062463 80.652463) (width 0.4) (layer F.Cu) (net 8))
 (segment (start 186.062463 80.652463) (end 185.42 80.01) (width 0.4) (layer F.Cu) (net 8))
 (segment (start 185.42 80.01) (end 166.37 80.01) (width 0.4) (layer F.Cu) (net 8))
 (segment (start 166.37 80.01) (end 165.735 79.375) (width 0.4) (layer F.Cu) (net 8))
 (segment (start 165.735 79.375) (end 165.735 76.835) (width 0.4) (layer F.Cu) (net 8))
 (via (at 165.735 76.835) (size 1.3) (drill 0.7) (layers F.Cu B.Cu) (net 8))
 (segment (start 165.735 76.835) (end 165.735 81.28) (width 0.4) (layer B.Cu) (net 8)))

